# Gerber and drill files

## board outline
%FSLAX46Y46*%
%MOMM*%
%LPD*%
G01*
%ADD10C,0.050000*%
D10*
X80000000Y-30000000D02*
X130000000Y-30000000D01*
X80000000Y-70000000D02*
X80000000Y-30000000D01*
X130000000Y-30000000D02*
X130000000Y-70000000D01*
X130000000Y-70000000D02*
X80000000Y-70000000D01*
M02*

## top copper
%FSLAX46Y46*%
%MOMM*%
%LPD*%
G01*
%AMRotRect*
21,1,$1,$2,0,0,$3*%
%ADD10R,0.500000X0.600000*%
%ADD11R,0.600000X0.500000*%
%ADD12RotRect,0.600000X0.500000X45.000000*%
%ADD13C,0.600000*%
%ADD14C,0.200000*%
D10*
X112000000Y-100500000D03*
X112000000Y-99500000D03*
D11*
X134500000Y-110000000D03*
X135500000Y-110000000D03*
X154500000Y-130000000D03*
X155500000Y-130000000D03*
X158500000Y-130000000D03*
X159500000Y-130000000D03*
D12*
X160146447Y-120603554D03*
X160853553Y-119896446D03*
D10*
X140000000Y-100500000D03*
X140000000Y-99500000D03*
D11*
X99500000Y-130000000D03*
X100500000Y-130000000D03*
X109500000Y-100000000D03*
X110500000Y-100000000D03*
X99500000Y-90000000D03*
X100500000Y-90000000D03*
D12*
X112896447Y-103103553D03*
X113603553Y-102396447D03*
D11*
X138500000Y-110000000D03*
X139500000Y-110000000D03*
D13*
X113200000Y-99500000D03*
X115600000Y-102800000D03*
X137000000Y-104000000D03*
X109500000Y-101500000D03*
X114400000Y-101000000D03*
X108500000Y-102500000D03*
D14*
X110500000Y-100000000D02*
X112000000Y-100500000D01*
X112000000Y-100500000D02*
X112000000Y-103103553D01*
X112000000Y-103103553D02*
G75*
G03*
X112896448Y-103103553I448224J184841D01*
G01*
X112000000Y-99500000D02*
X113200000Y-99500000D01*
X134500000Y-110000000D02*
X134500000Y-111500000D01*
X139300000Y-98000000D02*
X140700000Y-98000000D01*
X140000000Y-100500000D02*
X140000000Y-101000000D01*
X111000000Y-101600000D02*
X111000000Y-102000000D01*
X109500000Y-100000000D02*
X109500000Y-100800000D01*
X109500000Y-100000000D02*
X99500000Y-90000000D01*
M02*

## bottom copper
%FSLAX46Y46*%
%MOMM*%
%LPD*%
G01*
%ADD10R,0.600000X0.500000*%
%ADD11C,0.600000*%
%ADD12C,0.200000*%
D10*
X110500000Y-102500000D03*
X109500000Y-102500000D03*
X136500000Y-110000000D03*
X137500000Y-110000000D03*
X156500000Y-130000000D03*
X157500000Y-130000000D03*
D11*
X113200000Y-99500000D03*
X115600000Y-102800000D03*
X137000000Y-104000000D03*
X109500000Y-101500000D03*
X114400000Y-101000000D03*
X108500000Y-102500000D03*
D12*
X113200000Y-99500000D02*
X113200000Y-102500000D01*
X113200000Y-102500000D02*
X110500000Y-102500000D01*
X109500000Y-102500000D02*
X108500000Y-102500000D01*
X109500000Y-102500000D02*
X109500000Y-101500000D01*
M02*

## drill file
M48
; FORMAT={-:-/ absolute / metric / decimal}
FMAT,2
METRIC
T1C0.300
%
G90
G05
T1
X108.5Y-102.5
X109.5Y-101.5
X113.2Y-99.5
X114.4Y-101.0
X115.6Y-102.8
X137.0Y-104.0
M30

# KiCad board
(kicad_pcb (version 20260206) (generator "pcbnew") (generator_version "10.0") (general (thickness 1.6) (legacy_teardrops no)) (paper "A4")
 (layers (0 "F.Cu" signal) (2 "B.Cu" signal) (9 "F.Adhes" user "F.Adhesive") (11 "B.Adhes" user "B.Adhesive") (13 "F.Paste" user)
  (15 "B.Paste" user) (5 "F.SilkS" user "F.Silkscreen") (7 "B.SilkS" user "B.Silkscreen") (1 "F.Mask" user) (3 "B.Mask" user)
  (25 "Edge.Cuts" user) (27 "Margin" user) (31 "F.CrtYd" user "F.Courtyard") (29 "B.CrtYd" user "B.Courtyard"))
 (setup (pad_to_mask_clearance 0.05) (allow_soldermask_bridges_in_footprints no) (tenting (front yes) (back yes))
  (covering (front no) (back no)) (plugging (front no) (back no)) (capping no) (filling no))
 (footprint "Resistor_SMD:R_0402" (layer "F.Cu") (at 112 100 90)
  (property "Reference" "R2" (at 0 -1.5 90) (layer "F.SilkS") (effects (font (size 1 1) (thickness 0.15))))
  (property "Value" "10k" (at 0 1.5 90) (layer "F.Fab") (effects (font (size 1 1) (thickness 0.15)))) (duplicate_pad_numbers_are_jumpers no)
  (pad "1" smd rect (at -0.5 0 90) (size 0.6 0.5) (layers "F.Cu" "F.Mask" "F.Paste") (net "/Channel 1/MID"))
  (pad "2" smd rect (at 0.5 0 90) (size 0.6 0.5) (layers "F.Cu" "F.Mask" "F.Paste") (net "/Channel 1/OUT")))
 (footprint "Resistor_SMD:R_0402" (layer "F.Cu") (at 135 110)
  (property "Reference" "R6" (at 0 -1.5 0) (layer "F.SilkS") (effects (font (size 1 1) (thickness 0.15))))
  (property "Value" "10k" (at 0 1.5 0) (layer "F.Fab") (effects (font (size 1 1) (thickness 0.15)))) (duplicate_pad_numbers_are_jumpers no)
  (pad "1" smd rect (at -0.5 0) (size 0.6 0.5) (layers "F.Cu" "F.Mask" "F.Paste") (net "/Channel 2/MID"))
  (pad "2" smd rect (at 0.5 0) (size 0.6 0.5) (layers "F.Cu" "F.Mask" "F.Paste") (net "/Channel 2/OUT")))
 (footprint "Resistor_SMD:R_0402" (layer "F.Cu") (at 155 130)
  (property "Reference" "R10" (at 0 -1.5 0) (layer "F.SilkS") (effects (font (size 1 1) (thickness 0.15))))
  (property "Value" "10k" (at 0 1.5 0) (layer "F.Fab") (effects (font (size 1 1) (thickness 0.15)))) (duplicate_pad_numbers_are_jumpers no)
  (pad "1" smd rect (at -0.5 0) (size 0.6 0.5) (layers "F.Cu" "F.Mask" "F.Paste") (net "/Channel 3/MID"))
  (pad "2" smd rect (at 0.5 0) (size 0.6 0.5) (layers "F.Cu" "F.Mask" "F.Paste") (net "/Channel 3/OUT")))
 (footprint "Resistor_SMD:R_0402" (layer "F.Cu") (at 159 130)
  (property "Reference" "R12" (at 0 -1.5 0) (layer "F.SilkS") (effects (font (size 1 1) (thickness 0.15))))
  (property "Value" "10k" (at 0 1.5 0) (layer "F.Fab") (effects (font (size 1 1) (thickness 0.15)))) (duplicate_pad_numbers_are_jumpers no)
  (pad "1" smd rect (at -0.5 0) (size 0.6 0.5) (layers "F.Cu" "F.Mask" "F.Paste") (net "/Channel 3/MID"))
  (pad "2" smd rect (at 0.5 0) (size 0.6 0.5) (layers "F.Cu" "F.Mask" "F.Paste") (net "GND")))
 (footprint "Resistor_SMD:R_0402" (layer "F.Cu") (at 160.5 120.25 45)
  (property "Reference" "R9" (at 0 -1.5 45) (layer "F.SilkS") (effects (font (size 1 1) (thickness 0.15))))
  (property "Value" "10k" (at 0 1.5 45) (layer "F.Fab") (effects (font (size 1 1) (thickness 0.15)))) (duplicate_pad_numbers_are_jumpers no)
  (pad "1" smd rect (at -0.5 0.000001 45) (size 0.6 0.5) (layers "F.Cu" "F.Mask" "F.Paste") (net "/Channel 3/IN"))
  (pad "2" smd rect (at 0.5 -0.000001 45) (size 0.6 0.5) (layers "F.Cu" "F.Mask" "F.Paste") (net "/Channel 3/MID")))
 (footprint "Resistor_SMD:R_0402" (layer "F.Cu") (at 140 100 90)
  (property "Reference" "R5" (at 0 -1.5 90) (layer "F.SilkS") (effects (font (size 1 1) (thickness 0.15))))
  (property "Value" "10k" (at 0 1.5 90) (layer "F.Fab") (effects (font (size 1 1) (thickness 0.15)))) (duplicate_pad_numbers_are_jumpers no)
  (pad "1" smd rect (at -0.5 0 90) (size 0.6 0.5) (layers "F.Cu" "F.Mask" "F.Paste") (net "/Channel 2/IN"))
  (pad "2" smd rect (at 0.5 0 90) (size 0.6 0.5) (layers "F.Cu" "F.Mask" "F.Paste") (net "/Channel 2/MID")))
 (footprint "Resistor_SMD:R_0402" (layer "F.Cu") (at 100 130)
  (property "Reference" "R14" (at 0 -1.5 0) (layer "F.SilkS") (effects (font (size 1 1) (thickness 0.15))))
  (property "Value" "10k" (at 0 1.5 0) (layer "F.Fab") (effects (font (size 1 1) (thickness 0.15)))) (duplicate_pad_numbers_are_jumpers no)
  (pad "1" smd rect (at -0.5 0) (size 0.6 0.5) (layers "F.Cu" "F.Mask" "F.Paste") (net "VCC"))
  (pad "2" smd rect (at 0.5 0) (size 0.6 0.5) (layers "F.Cu" "F.Mask" "F.Paste") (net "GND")))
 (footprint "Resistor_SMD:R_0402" (layer "F.Cu") (at 110 100)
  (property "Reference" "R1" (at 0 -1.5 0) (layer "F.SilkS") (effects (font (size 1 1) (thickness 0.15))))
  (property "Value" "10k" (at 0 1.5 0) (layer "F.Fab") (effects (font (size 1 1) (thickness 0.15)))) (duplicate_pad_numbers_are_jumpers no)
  (pad "1" smd rect (at -0.5 0) (size 0.6 0.5) (layers "F.Cu" "F.Mask" "F.Paste") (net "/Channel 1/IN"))
  (pad "2" smd rect (at 0.5 0) (size 0.6 0.5) (layers "F.Cu" "F.Mask" "F.Paste") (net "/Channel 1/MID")))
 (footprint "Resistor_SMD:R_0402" (layer "F.Cu") (at 100 90)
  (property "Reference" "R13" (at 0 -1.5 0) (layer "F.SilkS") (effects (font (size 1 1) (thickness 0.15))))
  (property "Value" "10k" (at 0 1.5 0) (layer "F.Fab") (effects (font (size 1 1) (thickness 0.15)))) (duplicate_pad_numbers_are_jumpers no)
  (pad "1" smd rect (at -0.5 0) (size 0.6 0.5) (layers "F.Cu" "F.Mask" "F.Paste") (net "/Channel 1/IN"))
  (pad "2" smd rect (at 0.5 0) (size 0.6 0.5) (layers "F.Cu" "F.Mask" "F.Paste") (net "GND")))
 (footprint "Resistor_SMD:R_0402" (layer "F.Cu") (at 113.25 102.75 45)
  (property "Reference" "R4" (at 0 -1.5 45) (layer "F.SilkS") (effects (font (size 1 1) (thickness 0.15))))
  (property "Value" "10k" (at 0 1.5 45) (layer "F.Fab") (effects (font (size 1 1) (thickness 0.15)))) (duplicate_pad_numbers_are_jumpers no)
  (pad "1" smd rect (at -0.499999 0 45) (size 0.6 0.5) (layers "F.Cu" "F.Mask" "F.Paste") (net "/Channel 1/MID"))
  (pad "2" smd rect (at 0.499999 0 45) (size 0.6 0.5) (layers "F.Cu" "F.Mask" "F.Paste") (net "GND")))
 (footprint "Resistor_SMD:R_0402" (layer "F.Cu") (at 139 110)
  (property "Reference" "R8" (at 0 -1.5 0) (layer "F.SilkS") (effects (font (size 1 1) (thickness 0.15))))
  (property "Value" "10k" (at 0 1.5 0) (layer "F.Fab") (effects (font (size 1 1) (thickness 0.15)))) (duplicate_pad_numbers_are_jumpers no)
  (pad "1" smd rect (at -0.5 0) (size 0.6 0.5) (layers "F.Cu" "F.Mask" "F.Paste") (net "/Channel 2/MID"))
  (pad "2" smd rect (at 0.5 0) (size 0.6 0.5) (layers "F.Cu" "F.Mask" "F.Paste") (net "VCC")))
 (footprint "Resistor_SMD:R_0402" (layer "B.Cu") (at 110 102.5 180)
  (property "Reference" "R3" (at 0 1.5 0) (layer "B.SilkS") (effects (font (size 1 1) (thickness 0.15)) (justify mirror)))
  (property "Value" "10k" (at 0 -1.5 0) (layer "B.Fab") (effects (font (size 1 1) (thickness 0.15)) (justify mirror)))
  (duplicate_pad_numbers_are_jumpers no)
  (pad "1" smd rect (at -0.5 0 180) (size 0.6 0.5) (layers "B.Cu" "B.Mask" "B.Paste") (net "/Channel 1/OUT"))
  (pad "2" smd rect (at 0.5 0 180) (size 0.6 0.5) (layers "B.Cu" "B.Mask" "B.Paste") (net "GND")))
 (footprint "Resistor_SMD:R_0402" (layer "B.Cu") (at 137 110)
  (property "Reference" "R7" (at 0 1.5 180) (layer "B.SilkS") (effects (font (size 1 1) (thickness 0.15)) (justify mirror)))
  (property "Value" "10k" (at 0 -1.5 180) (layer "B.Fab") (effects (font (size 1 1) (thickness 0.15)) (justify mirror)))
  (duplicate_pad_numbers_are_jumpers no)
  (pad "1" smd rect (at -0.5 0) (size 0.6 0.5) (layers "B.Cu" "B.Mask" "B.Paste") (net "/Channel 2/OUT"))
  (pad "2" smd rect (at 0.5 0) (size 0.6 0.5) (layers "B.Cu" "B.Mask" "B.Paste") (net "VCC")))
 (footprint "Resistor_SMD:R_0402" (layer "B.Cu") (at 157 130)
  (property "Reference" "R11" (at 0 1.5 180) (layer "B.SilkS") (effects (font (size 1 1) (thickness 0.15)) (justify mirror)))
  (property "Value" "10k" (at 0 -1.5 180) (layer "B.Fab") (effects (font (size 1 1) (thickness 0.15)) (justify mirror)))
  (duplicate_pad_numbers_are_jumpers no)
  (pad "1" smd rect (at -0.5 0) (size 0.6 0.5) (layers "B.Cu" "B.Mask" "B.Paste") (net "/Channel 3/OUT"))
  (pad "2" smd rect (at 0.5 0) (size 0.6 0.5) (layers "B.Cu" "B.Mask" "B.Paste") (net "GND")))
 (gr_line (start 80 30) (end 130 30) (stroke (width 0.05) (type default)) (layer "Edge.Cuts"))
 (gr_line (start 80 70) (end 80 30) (stroke (width 0.05) (type default)) (layer "Edge.Cuts"))
 (gr_line (start 130 30) (end 130 70) (stroke (width 0.05) (type default)) (layer "Edge.Cuts"))
 (gr_line (start 130 70) (end 80 70) (stroke (width 0.05) (type default)) (layer "Edge.Cuts"))
 (segment (start 110.5 100) (end 112 100.5) (width 0.2) (locked yes) (layer "F.Cu") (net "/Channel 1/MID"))
 (segment (start 112 100.5) (end 112 103.103553) (width 0.2) (layer "F.Cu") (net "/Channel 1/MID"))
 (arc (start 112 103.103553) (mid 112.448223 103.403553) (end 112.896447 103.103553) (width 0.2) (layer "F.Cu") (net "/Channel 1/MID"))
 (segment (start 112 99.5) (end 113.2 99.5) (width 0.2) (layer "F.Cu") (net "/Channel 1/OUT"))
 (via (at 113.2 99.5) (size 0.6) (drill 0.3) (layers "F.Cu" "B.Cu") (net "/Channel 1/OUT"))
 (segment (start 113.2 99.5) (end 113.2 102.5) (width 0.2) (layer "B.Cu") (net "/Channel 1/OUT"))
 (segment (start 113.2 102.5) (end 110.5 102.5) (width 0.2) (layer "B.Cu") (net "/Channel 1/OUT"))
 (segment (start 134.5 110) (end 134.5 111.5) (width 0.2) (layer "F.Cu") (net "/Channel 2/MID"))
 (segment (start 139.3 98) (end 140.7 98) (width 0.2) (layer "F.Cu") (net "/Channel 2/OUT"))
 (via (at 115.6 102.8) (size 0.6) (drill 0.3) (layers "F.Cu" "B.Cu") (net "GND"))
 (via (at 137 104) (size 0.6) (drill 0.3) (layers "F.Cu" "B.Cu") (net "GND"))
 (via (at 109.5 101.5) (size 0.6) (drill 0.3) (layers "F.Cu" "B.Cu") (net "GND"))
 (via (at 114.4 101) (size 0.6) (drill 0.3) (layers "F.Cu" "B.Cu") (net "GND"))
 (via (at 108.5 102.5) (size 0.6) (drill 0.3) (layers "F.Cu" "B.Cu") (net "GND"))
 (segment (start 109.5 102.5) (end 108.5 102.5) (width 0.2) (layer "B.Cu") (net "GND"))
 (segment (start 109.5 102.5) (end 109.5 101.5) (width 0.2) (layer "B.Cu") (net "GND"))
 (segment (start 140 100.5) (end 140 101) (width 0.2) (layer "F.Cu") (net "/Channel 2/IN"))
 (segment (start 111 101.6) (end 111 102) (width 0.2) (layer "F.Cu") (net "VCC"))
 (segment (start 109.5 100) (end 109.5 100.8) (width 0.2) (layer "F.Cu") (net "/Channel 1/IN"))
 (segment (start 109.5 100) (end 99.5 90) (width 0.2) (layer "F.Cu") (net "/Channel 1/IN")))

